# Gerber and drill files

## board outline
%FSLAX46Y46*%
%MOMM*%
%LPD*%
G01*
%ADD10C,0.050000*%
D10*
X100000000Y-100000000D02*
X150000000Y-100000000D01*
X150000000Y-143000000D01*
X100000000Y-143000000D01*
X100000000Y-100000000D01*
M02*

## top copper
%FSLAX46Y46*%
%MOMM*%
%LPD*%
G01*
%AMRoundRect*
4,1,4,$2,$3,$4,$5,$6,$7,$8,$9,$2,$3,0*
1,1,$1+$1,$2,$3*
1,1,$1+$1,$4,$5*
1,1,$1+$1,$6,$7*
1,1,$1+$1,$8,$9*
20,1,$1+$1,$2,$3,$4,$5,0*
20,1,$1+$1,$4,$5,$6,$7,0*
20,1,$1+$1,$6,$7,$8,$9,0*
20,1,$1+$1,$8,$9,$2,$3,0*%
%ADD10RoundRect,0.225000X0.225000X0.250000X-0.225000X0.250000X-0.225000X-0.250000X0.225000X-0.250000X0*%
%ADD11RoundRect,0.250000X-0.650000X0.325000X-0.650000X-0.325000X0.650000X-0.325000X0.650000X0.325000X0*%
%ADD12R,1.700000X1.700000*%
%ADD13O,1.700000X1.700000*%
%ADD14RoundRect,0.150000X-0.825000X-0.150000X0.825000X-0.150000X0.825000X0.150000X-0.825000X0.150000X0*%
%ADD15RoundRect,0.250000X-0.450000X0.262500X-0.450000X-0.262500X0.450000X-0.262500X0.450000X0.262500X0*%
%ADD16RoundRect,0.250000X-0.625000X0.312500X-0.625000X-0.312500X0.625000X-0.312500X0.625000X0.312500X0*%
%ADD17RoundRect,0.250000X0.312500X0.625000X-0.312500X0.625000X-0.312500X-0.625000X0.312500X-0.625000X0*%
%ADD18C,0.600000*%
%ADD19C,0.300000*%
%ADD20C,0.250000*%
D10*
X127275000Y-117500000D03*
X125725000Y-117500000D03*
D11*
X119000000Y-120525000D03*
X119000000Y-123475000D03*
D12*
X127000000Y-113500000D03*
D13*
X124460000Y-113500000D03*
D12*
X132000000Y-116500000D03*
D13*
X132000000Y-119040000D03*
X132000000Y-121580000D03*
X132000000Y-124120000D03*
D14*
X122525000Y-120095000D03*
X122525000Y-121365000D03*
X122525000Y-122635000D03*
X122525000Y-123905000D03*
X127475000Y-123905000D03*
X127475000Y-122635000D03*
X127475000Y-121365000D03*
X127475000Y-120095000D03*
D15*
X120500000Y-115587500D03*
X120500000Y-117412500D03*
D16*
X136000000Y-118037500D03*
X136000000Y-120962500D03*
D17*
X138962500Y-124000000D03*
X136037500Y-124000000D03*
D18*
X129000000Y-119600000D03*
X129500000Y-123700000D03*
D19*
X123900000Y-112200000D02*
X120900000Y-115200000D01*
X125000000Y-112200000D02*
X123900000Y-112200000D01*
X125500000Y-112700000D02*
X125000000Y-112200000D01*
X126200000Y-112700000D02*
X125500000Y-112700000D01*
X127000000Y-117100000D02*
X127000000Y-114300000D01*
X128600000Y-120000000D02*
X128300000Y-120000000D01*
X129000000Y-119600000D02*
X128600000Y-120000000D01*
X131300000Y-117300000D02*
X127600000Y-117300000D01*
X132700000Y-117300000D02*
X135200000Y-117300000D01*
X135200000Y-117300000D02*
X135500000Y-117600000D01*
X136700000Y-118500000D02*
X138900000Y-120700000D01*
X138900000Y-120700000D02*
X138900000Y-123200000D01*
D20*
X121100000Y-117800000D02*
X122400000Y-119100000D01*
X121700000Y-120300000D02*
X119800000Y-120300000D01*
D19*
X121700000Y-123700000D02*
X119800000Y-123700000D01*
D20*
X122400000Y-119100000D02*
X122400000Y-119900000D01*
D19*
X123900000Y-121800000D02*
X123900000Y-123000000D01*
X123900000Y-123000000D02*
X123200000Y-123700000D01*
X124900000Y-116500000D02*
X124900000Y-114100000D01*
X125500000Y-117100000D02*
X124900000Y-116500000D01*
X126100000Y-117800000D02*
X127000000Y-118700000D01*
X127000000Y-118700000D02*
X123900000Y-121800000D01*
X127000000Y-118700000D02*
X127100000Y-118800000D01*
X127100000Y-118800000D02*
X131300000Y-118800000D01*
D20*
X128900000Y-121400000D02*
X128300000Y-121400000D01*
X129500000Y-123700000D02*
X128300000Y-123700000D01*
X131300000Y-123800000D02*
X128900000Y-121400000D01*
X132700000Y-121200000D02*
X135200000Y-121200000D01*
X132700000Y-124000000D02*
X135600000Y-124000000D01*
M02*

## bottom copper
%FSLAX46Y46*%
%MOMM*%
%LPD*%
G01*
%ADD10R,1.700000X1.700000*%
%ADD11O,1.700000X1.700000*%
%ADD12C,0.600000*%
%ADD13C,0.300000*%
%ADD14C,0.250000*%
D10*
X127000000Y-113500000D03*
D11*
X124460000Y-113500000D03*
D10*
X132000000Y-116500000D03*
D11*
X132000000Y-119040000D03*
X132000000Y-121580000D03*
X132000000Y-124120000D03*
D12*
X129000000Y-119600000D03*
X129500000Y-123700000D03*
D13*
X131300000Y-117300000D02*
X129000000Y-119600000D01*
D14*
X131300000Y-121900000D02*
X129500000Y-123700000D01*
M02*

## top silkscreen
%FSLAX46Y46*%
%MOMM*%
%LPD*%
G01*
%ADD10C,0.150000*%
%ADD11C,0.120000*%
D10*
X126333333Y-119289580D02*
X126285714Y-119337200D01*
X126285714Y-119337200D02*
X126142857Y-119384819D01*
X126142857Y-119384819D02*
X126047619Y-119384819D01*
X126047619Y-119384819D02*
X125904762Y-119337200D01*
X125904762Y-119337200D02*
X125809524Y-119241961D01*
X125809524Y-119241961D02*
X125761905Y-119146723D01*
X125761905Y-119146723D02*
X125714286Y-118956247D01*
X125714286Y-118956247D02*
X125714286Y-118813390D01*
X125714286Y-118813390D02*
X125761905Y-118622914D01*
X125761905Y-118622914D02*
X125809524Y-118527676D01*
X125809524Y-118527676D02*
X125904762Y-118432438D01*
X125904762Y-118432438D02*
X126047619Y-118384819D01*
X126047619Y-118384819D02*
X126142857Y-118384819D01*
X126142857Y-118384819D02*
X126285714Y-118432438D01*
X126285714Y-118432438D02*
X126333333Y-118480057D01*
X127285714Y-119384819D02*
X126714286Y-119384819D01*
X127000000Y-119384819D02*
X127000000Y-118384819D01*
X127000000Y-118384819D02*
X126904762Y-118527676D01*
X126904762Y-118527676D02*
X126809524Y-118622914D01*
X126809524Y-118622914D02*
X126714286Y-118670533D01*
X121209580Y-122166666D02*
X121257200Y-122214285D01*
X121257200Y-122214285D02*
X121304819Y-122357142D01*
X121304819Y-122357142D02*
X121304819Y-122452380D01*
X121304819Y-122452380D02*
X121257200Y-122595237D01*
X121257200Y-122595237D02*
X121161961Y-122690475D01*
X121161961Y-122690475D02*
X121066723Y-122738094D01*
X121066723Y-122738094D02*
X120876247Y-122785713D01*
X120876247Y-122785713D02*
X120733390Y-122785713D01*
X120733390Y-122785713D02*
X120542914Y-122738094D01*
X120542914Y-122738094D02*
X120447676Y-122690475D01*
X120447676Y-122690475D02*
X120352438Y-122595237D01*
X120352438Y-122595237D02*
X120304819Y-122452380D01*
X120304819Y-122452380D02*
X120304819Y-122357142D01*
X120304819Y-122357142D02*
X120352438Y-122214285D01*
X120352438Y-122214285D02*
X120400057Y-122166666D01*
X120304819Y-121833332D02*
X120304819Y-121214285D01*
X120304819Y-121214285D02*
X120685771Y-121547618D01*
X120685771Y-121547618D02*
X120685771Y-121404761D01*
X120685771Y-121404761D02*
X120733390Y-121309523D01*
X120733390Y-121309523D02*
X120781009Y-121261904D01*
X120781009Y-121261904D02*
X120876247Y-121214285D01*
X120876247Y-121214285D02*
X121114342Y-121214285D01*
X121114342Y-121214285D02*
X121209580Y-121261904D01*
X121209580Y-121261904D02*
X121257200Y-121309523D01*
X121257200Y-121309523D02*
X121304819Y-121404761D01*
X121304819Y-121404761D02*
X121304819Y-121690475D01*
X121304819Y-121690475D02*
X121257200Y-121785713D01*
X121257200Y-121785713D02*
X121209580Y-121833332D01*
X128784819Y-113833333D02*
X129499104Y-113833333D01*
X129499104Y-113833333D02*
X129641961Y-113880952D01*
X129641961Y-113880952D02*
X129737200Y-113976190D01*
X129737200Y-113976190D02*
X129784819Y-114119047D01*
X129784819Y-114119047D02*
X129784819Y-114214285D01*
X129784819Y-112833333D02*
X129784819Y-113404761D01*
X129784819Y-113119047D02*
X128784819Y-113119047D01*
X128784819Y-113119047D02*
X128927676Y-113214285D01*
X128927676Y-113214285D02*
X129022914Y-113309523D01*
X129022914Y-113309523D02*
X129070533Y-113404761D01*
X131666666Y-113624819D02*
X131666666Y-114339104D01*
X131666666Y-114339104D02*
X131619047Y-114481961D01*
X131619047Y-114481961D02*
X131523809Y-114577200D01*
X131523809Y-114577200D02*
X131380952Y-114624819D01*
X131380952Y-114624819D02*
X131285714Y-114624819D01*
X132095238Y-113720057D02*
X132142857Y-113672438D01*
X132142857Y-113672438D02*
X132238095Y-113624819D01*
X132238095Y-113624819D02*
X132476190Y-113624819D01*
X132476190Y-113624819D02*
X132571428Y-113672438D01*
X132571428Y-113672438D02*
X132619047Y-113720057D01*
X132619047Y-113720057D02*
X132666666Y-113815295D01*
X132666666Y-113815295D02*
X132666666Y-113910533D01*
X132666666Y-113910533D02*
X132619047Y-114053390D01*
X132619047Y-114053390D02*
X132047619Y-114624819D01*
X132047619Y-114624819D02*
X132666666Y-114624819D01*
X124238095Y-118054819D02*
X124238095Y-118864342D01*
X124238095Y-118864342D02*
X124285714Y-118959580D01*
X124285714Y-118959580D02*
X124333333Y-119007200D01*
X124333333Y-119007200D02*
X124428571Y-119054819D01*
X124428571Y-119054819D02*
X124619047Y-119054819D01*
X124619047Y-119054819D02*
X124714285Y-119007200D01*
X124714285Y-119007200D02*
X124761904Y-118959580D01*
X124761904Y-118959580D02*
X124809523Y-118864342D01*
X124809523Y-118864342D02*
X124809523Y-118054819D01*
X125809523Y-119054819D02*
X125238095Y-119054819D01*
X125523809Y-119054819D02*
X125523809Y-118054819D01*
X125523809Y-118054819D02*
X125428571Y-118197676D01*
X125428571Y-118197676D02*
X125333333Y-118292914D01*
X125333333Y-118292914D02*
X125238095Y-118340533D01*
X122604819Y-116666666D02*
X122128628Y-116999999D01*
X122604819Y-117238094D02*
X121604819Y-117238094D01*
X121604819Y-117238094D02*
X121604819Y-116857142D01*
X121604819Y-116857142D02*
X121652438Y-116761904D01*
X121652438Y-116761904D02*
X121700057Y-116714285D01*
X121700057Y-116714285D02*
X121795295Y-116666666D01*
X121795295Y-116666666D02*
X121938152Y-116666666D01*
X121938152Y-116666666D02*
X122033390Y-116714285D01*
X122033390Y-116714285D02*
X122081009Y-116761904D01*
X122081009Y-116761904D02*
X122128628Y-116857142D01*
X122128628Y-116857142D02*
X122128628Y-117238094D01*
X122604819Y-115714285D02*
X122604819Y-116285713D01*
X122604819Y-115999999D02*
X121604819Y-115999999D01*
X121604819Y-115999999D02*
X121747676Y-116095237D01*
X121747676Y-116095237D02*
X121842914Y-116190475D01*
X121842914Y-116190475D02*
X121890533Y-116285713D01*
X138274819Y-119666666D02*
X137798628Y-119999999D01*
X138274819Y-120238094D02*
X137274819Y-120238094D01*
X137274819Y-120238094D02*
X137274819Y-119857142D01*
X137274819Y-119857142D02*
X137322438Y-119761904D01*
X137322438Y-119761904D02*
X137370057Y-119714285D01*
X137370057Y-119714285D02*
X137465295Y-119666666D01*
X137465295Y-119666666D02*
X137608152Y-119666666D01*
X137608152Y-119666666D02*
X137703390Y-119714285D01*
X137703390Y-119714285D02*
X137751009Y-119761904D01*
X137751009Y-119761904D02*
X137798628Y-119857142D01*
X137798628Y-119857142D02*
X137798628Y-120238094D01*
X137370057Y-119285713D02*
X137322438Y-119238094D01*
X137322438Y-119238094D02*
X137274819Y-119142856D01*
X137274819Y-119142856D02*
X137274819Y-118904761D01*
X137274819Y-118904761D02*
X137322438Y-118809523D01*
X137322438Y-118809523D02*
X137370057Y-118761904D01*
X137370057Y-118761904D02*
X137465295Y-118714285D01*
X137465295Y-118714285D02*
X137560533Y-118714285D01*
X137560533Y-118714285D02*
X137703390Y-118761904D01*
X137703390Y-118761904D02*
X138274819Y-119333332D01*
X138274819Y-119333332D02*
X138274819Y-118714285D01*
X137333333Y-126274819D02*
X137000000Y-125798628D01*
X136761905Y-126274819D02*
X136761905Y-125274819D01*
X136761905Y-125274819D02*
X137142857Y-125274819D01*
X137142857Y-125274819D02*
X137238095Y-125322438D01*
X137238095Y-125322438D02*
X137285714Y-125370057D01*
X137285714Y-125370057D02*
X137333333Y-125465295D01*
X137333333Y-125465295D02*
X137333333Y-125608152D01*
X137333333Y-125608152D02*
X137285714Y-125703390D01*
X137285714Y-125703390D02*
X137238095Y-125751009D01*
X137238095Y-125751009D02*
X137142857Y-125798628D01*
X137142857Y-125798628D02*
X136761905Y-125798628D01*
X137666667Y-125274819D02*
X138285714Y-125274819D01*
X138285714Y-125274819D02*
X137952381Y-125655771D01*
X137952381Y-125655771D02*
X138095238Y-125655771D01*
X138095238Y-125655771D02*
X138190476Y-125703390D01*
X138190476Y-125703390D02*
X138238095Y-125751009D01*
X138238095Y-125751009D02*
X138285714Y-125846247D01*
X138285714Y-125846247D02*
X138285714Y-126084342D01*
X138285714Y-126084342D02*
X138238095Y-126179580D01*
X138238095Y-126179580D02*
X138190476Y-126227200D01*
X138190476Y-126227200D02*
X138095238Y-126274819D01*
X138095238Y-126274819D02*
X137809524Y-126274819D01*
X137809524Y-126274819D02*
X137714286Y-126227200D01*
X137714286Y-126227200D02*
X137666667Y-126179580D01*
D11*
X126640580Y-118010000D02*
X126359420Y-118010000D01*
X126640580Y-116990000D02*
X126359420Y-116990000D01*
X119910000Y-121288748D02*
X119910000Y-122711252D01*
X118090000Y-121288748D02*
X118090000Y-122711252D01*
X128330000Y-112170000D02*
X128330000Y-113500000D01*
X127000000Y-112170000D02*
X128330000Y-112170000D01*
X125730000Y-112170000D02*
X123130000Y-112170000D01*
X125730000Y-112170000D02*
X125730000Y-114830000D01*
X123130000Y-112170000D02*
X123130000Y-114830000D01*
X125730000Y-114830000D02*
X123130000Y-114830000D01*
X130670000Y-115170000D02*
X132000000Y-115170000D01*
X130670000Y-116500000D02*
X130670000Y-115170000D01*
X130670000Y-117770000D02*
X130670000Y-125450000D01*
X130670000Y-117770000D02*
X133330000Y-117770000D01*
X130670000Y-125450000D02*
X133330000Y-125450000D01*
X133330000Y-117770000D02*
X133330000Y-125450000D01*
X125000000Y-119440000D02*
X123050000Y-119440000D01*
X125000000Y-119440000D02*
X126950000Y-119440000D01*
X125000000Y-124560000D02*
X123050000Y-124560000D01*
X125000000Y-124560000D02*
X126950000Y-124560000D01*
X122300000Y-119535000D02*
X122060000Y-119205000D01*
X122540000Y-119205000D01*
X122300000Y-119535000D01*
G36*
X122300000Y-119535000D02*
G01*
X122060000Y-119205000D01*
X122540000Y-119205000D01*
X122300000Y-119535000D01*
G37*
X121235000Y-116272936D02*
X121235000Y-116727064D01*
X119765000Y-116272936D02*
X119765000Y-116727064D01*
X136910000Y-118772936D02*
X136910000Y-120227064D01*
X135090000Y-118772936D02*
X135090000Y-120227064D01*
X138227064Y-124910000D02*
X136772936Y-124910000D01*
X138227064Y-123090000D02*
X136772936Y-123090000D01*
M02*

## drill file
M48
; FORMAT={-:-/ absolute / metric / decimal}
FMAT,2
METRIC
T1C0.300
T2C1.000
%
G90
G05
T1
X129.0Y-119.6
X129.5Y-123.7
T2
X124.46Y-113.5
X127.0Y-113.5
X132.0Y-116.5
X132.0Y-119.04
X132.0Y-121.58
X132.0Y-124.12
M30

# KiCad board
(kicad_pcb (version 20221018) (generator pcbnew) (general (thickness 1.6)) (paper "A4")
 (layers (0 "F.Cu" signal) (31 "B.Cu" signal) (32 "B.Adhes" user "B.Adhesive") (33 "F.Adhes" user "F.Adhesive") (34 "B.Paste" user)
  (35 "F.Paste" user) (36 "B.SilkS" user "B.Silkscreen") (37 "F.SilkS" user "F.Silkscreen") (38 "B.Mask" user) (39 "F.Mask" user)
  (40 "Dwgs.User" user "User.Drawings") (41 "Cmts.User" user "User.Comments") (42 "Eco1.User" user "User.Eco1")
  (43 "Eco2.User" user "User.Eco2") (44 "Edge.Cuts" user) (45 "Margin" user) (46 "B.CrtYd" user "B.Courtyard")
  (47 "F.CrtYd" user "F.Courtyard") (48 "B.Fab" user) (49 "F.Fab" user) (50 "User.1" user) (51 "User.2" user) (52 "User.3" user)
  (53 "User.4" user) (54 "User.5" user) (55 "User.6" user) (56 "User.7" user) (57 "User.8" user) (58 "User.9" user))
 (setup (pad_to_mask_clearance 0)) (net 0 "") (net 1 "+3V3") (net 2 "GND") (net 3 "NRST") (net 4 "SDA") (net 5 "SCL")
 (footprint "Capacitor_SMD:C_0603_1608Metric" (layer "F.Cu") (at 126.5 117.5 180)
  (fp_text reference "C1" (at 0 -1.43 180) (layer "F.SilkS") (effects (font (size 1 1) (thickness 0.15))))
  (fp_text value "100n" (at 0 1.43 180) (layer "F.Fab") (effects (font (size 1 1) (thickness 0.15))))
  (fp_line (start -0.14058 -0.51) (end 0.14058 -0.51) (stroke (width 0.12) (type solid)) (layer "F.SilkS"))
  (fp_line (start -0.14058 0.51) (end 0.14058 0.51) (stroke (width 0.12) (type solid)) (layer "F.SilkS"))
  (pad "1" smd roundrect (at -0.775 0 180) (size 0.9 0.95) (layers "F.Cu" "F.Paste" "F.Mask") (roundrect_rratio 0.25) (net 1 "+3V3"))
  (pad "2" smd roundrect (at 0.775 0 180) (size 0.9 0.95) (layers "F.Cu" "F.Paste" "F.Mask") (roundrect_rratio 0.25) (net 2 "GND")))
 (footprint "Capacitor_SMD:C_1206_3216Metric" (layer "F.Cu") (at 119 122 -90)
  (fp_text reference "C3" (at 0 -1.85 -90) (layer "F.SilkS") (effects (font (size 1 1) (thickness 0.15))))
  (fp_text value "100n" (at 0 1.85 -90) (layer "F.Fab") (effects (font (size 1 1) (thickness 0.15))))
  (fp_line (start -0.711252 -0.91) (end 0.711252 -0.91) (stroke (width 0.12) (type solid)) (layer "F.SilkS"))
  (fp_line (start -0.711252 0.91) (end 0.711252 0.91) (stroke (width 0.12) (type solid)) (layer "F.SilkS"))
  (pad "1" smd roundrect (at -1.475 0 270) (size 1.15 1.8) (layers "F.Cu" "F.Paste" "F.Mask") (roundrect_rratio 0.217391) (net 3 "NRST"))
  (pad "2" smd roundrect (at 1.475 0 270) (size 1.15 1.8) (layers "F.Cu" "F.Paste" "F.Mask") (roundrect_rratio 0.217391) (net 2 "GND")))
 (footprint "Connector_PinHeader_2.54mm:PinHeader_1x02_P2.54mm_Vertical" (layer "F.Cu") (at 127 113.5 -90)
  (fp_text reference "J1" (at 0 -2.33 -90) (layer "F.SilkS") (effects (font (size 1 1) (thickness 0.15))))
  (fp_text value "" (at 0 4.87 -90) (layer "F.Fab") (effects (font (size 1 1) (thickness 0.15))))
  (fp_line (start -1.33 -1.33) (end 0 -1.33) (stroke (width 0.12) (type solid)) (layer "F.SilkS"))
  (fp_line (start -1.33 0) (end -1.33 -1.33) (stroke (width 0.12) (type solid)) (layer "F.SilkS"))
  (fp_line (start -1.33 1.27) (end -1.33 3.87) (stroke (width 0.12) (type solid)) (layer "F.SilkS"))
  (fp_line (start -1.33 1.27) (end 1.33 1.27) (stroke (width 0.12) (type solid)) (layer "F.SilkS"))
  (fp_line (start -1.33 3.87) (end 1.33 3.87) (stroke (width 0.12) (type solid)) (layer "F.SilkS"))
  (fp_line (start 1.33 1.27) (end 1.33 3.87) (stroke (width 0.12) (type solid)) (layer "F.SilkS"))
  (pad "1" thru_hole rect (at 0 0 270) (size 1.7 1.7) (drill 1) (layers "*.Cu" "*.Mask") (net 1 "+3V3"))
  (pad "2" thru_hole oval (at 0 2.54 270) (size 1.7 1.7) (drill 1) (layers "*.Cu" "*.Mask") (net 2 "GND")))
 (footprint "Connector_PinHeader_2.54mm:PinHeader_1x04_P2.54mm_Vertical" (layer "F.Cu") (at 132 116.5)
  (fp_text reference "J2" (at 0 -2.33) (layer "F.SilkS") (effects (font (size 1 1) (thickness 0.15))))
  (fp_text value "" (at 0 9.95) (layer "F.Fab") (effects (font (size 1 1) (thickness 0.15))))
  (fp_line (start -1.33 -1.33) (end 0 -1.33) (stroke (width 0.12) (type solid)) (layer "F.SilkS"))
  (fp_line (start -1.33 0) (end -1.33 -1.33) (stroke (width 0.12) (type solid)) (layer "F.SilkS"))
  (fp_line (start -1.33 1.27) (end -1.33 8.95) (stroke (width 0.12) (type solid)) (layer "F.SilkS"))
  (fp_line (start -1.33 1.27) (end 1.33 1.27) (stroke (width 0.12) (type solid)) (layer "F.SilkS"))
  (fp_line (start -1.33 8.95) (end 1.33 8.95) (stroke (width 0.12) (type solid)) (layer "F.SilkS"))
  (fp_line (start 1.33 1.27) (end 1.33 8.95) (stroke (width 0.12) (type solid)) (layer "F.SilkS"))
  (pad "1" thru_hole rect (at 0 0) (size 1.7 1.7) (drill 1) (layers "*.Cu" "*.Mask") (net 1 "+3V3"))
  (pad "2" thru_hole oval (at 0 2.54) (size 1.7 1.7) (drill 1) (layers "*.Cu" "*.Mask") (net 2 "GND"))
  (pad "3" thru_hole oval (at 0 5.08) (size 1.7 1.7) (drill 1) (layers "*.Cu" "*.Mask") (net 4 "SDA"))
  (pad "4" thru_hole oval (at 0 7.62) (size 1.7 1.7) (drill 1) (layers "*.Cu" "*.Mask") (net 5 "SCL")))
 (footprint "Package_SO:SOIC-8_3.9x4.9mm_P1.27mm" (layer "F.Cu") (at 125 122)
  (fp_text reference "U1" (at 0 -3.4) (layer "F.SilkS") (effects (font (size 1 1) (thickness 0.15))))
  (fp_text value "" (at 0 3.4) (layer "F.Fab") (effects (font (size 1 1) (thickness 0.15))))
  (fp_line (start 0 -2.56) (end -1.95 -2.56) (stroke (width 0.12) (type solid)) (layer "F.SilkS"))
  (fp_line (start 0 -2.56) (end 1.95 -2.56) (stroke (width 0.12) (type solid)) (layer "F.SilkS"))
  (fp_line (start 0 2.56) (end -1.95 2.56) (stroke (width 0.12) (type solid)) (layer "F.SilkS"))
  (fp_line (start 0 2.56) (end 1.95 2.56) (stroke (width 0.12) (type solid)) (layer "F.SilkS"))
  (fp_poly
   (pts (xy -2.7 -2.465) (xy -2.94 -2.795) (xy -2.46 -2.795) (xy -2.7 -2.465)) (stroke (width 0.12) (type solid)) (fill solid)
   (layer "F.SilkS"))
  (pad "1" smd roundrect (at -2.475 -1.905) (size 1.95 0.6) (layers "F.Cu" "F.Paste" "F.Mask") (roundrect_rratio 0.25) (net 3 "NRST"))
  (pad "2" smd roundrect (at -2.475 -0.635) (size 1.95 0.6) (layers "F.Cu" "F.Paste" "F.Mask") (roundrect_rratio 0.25))
  (pad "3" smd roundrect (at -2.475 0.635) (size 1.95 0.6) (layers "F.Cu" "F.Paste" "F.Mask") (roundrect_rratio 0.25))
  (pad "4" smd roundrect (at -2.475 1.905) (size 1.95 0.6) (layers "F.Cu" "F.Paste" "F.Mask") (roundrect_rratio 0.25) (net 2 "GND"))
  (pad "5" smd roundrect (at 2.475 1.905) (size 1.95 0.6) (layers "F.Cu" "F.Paste" "F.Mask") (roundrect_rratio 0.25) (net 4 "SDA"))
  (pad "6" smd roundrect (at 2.475 0.635) (size 1.95 0.6) (layers "F.Cu" "F.Paste" "F.Mask") (roundrect_rratio 0.25))
  (pad "7" smd roundrect (at 2.475 -0.635) (size 1.95 0.6) (layers "F.Cu" "F.Paste" "F.Mask") (roundrect_rratio 0.25) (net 5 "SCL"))
  (pad "8" smd roundrect (at 2.475 -1.905) (size 1.95 0.6) (layers "F.Cu" "F.Paste" "F.Mask") (roundrect_rratio 0.25) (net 1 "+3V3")))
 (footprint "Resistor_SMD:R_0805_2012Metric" (layer "F.Cu") (at 120.5 116.5 -90)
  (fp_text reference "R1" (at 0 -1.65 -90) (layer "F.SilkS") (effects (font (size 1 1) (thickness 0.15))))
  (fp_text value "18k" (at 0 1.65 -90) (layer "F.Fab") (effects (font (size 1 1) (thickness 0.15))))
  (fp_line (start -0.227064 -0.735) (end 0.227064 -0.735) (stroke (width 0.12) (type solid)) (layer "F.SilkS"))
  (fp_line (start -0.227064 0.735) (end 0.227064 0.735) (stroke (width 0.12) (type solid)) (layer "F.SilkS"))
  (pad "1" smd roundrect (at -0.9125 0 270) (size 1.025 1.4) (layers "F.Cu" "F.Paste" "F.Mask") (roundrect_rratio 0.243902) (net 1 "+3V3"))
  (pad "2" smd roundrect (at 0.9125 0 270) (size 1.025 1.4) (layers "F.Cu" "F.Paste" "F.Mask") (roundrect_rratio 0.243902) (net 3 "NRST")))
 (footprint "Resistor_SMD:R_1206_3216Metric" (layer "F.Cu") (at 136 119.5 -90)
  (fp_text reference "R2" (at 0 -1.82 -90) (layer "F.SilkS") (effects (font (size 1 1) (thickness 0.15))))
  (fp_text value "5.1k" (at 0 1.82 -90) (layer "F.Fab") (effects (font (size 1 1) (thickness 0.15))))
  (fp_line (start -0.727064 -0.91) (end 0.727064 -0.91) (stroke (width 0.12) (type solid)) (layer "F.SilkS"))
  (fp_line (start -0.727064 0.91) (end 0.727064 0.91) (stroke (width 0.12) (type solid)) (layer "F.SilkS"))
  (pad "1" smd roundrect (at -1.4625 0 270) (size 1.125 1.75) (layers "F.Cu" "F.Paste" "F.Mask") (roundrect_rratio 0.222222) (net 1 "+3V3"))
  (pad "2" smd roundrect (at 1.4625 0 270) (size 1.125 1.75) (layers "F.Cu" "F.Paste" "F.Mask") (roundrect_rratio 0.222222) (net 4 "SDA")))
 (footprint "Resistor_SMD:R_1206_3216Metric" (layer "F.Cu") (at 137.5 124 180)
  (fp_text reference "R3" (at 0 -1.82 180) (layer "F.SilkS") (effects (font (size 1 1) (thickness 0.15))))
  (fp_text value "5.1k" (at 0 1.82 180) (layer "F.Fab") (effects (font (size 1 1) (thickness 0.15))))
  (fp_line (start -0.727064 -0.91) (end 0.727064 -0.91) (stroke (width 0.12) (type solid)) (layer "F.SilkS"))
  (fp_line (start -0.727064 0.91) (end 0.727064 0.91) (stroke (width 0.12) (type solid)) (layer "F.SilkS"))
  (pad "1" smd roundrect (at -1.4625 0 180) (size 1.125 1.75) (layers "F.Cu" "F.Paste" "F.Mask") (roundrect_rratio 0.222222) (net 1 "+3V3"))
  (pad "2" smd roundrect (at 1.4625 0 180) (size 1.125 1.75) (layers "F.Cu" "F.Paste" "F.Mask") (roundrect_rratio 0.222222) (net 5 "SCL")))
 (gr_rect (start 100 100) (end 150 143) (stroke (width 0.05) (type default)) (fill none) (layer "Edge.Cuts"))
 (segment (start 123.9 112.2) (end 120.9 115.2) (width 0.3) (layer "F.Cu") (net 1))
 (segment (start 125 112.2) (end 123.9 112.2) (width 0.3) (layer "F.Cu") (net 1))
 (segment (start 125.5 112.7) (end 125 112.2) (width 0.3) (layer "F.Cu") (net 1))
 (segment (start 126.2 112.7) (end 125.5 112.7) (width 0.3) (layer "F.Cu") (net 1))
 (segment (start 127 117.1) (end 127 114.3) (width 0.3) (layer "F.Cu") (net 1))
 (segment (start 128.6 120) (end 128.3 120) (width 0.3) (layer "F.Cu") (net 1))
 (segment (start 129 119.6) (end 128.6 120) (width 0.3) (layer "F.Cu") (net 1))
 (segment (start 131.3 117.3) (end 127.6 117.3) (width 0.3) (layer "F.Cu") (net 1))
 (segment (start 132.7 117.3) (end 135.2 117.3) (width 0.3) (layer "F.Cu") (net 1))
 (segment (start 135.2 117.3) (end 135.5 117.6) (width 0.3) (layer "F.Cu") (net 1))
 (segment (start 136.7 118.5) (end 138.9 120.7) (width 0.3) (layer "F.Cu") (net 1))
 (segment (start 138.9 120.7) (end 138.9 123.2) (width 0.3) (layer "F.Cu") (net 1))
 (via (at 129 119.6) (size 0.6) (drill 0.3) (layers "F.Cu" "B.Cu") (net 1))
 (segment (start 121.1 117.8) (end 122.4 119.1) (width 0.25) (layer "F.Cu") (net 3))
 (segment (start 121.7 120.3) (end 119.8 120.3) (width 0.25) (layer "F.Cu") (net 3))
 (segment (start 121.7 123.7) (end 119.8 123.7) (width 0.3) (layer "F.Cu") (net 2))
 (segment (start 122.4 119.1) (end 122.4 119.9) (width 0.25) (layer "F.Cu") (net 3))
 (segment (start 123.9 121.8) (end 123.9 123) (width 0.3) (layer "F.Cu") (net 2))
 (segment (start 123.9 123) (end 123.2 123.7) (width 0.3) (layer "F.Cu") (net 2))
 (segment (start 124.9 116.5) (end 124.9 114.1) (width 0.3) (layer "F.Cu") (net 2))
 (segment (start 125.5 117.1) (end 124.9 116.5) (width 0.3) (layer "F.Cu") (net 2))
 (segment (start 126.1 117.8) (end 127 118.7) (width 0.3) (layer "F.Cu") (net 2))
 (segment (start 127 118.7) (end 123.9 121.8) (width 0.3) (layer "F.Cu") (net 2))
 (segment (start 127 118.7) (end 127.1 118.8) (width 0.3) (layer "F.Cu") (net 2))
 (segment (start 127.1 118.8) (end 131.3 118.8) (width 0.3) (layer "F.Cu") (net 2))
 (segment (start 128.9 121.4) (end 128.3 121.4) (width 0.25) (layer "F.Cu") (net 5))
 (segment (start 129.5 123.7) (end 128.3 123.7) (width 0.25) (layer "F.Cu") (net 4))
 (segment (start 131.3 117.3) (end 129 119.6) (width 0.3) (layer "B.Cu") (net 1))
 (segment (start 131.3 123.8) (end 128.9 121.4) (width 0.25) (layer "F.Cu") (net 5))
 (segment (start 132.7 121.2) (end 135.2 121.2) (width 0.25) (layer "F.Cu") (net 4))
 (segment (start 132.7 124) (end 135.6 124) (width 0.25) (layer "F.Cu") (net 5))
 (via (at 129.5 123.7) (size 0.6) (drill 0.3) (layers "F.Cu" "B.Cu") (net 4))
 (segment (start 131.3 121.9) (end 129.5 123.7) (width 0.25) (layer "B.Cu") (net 4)))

